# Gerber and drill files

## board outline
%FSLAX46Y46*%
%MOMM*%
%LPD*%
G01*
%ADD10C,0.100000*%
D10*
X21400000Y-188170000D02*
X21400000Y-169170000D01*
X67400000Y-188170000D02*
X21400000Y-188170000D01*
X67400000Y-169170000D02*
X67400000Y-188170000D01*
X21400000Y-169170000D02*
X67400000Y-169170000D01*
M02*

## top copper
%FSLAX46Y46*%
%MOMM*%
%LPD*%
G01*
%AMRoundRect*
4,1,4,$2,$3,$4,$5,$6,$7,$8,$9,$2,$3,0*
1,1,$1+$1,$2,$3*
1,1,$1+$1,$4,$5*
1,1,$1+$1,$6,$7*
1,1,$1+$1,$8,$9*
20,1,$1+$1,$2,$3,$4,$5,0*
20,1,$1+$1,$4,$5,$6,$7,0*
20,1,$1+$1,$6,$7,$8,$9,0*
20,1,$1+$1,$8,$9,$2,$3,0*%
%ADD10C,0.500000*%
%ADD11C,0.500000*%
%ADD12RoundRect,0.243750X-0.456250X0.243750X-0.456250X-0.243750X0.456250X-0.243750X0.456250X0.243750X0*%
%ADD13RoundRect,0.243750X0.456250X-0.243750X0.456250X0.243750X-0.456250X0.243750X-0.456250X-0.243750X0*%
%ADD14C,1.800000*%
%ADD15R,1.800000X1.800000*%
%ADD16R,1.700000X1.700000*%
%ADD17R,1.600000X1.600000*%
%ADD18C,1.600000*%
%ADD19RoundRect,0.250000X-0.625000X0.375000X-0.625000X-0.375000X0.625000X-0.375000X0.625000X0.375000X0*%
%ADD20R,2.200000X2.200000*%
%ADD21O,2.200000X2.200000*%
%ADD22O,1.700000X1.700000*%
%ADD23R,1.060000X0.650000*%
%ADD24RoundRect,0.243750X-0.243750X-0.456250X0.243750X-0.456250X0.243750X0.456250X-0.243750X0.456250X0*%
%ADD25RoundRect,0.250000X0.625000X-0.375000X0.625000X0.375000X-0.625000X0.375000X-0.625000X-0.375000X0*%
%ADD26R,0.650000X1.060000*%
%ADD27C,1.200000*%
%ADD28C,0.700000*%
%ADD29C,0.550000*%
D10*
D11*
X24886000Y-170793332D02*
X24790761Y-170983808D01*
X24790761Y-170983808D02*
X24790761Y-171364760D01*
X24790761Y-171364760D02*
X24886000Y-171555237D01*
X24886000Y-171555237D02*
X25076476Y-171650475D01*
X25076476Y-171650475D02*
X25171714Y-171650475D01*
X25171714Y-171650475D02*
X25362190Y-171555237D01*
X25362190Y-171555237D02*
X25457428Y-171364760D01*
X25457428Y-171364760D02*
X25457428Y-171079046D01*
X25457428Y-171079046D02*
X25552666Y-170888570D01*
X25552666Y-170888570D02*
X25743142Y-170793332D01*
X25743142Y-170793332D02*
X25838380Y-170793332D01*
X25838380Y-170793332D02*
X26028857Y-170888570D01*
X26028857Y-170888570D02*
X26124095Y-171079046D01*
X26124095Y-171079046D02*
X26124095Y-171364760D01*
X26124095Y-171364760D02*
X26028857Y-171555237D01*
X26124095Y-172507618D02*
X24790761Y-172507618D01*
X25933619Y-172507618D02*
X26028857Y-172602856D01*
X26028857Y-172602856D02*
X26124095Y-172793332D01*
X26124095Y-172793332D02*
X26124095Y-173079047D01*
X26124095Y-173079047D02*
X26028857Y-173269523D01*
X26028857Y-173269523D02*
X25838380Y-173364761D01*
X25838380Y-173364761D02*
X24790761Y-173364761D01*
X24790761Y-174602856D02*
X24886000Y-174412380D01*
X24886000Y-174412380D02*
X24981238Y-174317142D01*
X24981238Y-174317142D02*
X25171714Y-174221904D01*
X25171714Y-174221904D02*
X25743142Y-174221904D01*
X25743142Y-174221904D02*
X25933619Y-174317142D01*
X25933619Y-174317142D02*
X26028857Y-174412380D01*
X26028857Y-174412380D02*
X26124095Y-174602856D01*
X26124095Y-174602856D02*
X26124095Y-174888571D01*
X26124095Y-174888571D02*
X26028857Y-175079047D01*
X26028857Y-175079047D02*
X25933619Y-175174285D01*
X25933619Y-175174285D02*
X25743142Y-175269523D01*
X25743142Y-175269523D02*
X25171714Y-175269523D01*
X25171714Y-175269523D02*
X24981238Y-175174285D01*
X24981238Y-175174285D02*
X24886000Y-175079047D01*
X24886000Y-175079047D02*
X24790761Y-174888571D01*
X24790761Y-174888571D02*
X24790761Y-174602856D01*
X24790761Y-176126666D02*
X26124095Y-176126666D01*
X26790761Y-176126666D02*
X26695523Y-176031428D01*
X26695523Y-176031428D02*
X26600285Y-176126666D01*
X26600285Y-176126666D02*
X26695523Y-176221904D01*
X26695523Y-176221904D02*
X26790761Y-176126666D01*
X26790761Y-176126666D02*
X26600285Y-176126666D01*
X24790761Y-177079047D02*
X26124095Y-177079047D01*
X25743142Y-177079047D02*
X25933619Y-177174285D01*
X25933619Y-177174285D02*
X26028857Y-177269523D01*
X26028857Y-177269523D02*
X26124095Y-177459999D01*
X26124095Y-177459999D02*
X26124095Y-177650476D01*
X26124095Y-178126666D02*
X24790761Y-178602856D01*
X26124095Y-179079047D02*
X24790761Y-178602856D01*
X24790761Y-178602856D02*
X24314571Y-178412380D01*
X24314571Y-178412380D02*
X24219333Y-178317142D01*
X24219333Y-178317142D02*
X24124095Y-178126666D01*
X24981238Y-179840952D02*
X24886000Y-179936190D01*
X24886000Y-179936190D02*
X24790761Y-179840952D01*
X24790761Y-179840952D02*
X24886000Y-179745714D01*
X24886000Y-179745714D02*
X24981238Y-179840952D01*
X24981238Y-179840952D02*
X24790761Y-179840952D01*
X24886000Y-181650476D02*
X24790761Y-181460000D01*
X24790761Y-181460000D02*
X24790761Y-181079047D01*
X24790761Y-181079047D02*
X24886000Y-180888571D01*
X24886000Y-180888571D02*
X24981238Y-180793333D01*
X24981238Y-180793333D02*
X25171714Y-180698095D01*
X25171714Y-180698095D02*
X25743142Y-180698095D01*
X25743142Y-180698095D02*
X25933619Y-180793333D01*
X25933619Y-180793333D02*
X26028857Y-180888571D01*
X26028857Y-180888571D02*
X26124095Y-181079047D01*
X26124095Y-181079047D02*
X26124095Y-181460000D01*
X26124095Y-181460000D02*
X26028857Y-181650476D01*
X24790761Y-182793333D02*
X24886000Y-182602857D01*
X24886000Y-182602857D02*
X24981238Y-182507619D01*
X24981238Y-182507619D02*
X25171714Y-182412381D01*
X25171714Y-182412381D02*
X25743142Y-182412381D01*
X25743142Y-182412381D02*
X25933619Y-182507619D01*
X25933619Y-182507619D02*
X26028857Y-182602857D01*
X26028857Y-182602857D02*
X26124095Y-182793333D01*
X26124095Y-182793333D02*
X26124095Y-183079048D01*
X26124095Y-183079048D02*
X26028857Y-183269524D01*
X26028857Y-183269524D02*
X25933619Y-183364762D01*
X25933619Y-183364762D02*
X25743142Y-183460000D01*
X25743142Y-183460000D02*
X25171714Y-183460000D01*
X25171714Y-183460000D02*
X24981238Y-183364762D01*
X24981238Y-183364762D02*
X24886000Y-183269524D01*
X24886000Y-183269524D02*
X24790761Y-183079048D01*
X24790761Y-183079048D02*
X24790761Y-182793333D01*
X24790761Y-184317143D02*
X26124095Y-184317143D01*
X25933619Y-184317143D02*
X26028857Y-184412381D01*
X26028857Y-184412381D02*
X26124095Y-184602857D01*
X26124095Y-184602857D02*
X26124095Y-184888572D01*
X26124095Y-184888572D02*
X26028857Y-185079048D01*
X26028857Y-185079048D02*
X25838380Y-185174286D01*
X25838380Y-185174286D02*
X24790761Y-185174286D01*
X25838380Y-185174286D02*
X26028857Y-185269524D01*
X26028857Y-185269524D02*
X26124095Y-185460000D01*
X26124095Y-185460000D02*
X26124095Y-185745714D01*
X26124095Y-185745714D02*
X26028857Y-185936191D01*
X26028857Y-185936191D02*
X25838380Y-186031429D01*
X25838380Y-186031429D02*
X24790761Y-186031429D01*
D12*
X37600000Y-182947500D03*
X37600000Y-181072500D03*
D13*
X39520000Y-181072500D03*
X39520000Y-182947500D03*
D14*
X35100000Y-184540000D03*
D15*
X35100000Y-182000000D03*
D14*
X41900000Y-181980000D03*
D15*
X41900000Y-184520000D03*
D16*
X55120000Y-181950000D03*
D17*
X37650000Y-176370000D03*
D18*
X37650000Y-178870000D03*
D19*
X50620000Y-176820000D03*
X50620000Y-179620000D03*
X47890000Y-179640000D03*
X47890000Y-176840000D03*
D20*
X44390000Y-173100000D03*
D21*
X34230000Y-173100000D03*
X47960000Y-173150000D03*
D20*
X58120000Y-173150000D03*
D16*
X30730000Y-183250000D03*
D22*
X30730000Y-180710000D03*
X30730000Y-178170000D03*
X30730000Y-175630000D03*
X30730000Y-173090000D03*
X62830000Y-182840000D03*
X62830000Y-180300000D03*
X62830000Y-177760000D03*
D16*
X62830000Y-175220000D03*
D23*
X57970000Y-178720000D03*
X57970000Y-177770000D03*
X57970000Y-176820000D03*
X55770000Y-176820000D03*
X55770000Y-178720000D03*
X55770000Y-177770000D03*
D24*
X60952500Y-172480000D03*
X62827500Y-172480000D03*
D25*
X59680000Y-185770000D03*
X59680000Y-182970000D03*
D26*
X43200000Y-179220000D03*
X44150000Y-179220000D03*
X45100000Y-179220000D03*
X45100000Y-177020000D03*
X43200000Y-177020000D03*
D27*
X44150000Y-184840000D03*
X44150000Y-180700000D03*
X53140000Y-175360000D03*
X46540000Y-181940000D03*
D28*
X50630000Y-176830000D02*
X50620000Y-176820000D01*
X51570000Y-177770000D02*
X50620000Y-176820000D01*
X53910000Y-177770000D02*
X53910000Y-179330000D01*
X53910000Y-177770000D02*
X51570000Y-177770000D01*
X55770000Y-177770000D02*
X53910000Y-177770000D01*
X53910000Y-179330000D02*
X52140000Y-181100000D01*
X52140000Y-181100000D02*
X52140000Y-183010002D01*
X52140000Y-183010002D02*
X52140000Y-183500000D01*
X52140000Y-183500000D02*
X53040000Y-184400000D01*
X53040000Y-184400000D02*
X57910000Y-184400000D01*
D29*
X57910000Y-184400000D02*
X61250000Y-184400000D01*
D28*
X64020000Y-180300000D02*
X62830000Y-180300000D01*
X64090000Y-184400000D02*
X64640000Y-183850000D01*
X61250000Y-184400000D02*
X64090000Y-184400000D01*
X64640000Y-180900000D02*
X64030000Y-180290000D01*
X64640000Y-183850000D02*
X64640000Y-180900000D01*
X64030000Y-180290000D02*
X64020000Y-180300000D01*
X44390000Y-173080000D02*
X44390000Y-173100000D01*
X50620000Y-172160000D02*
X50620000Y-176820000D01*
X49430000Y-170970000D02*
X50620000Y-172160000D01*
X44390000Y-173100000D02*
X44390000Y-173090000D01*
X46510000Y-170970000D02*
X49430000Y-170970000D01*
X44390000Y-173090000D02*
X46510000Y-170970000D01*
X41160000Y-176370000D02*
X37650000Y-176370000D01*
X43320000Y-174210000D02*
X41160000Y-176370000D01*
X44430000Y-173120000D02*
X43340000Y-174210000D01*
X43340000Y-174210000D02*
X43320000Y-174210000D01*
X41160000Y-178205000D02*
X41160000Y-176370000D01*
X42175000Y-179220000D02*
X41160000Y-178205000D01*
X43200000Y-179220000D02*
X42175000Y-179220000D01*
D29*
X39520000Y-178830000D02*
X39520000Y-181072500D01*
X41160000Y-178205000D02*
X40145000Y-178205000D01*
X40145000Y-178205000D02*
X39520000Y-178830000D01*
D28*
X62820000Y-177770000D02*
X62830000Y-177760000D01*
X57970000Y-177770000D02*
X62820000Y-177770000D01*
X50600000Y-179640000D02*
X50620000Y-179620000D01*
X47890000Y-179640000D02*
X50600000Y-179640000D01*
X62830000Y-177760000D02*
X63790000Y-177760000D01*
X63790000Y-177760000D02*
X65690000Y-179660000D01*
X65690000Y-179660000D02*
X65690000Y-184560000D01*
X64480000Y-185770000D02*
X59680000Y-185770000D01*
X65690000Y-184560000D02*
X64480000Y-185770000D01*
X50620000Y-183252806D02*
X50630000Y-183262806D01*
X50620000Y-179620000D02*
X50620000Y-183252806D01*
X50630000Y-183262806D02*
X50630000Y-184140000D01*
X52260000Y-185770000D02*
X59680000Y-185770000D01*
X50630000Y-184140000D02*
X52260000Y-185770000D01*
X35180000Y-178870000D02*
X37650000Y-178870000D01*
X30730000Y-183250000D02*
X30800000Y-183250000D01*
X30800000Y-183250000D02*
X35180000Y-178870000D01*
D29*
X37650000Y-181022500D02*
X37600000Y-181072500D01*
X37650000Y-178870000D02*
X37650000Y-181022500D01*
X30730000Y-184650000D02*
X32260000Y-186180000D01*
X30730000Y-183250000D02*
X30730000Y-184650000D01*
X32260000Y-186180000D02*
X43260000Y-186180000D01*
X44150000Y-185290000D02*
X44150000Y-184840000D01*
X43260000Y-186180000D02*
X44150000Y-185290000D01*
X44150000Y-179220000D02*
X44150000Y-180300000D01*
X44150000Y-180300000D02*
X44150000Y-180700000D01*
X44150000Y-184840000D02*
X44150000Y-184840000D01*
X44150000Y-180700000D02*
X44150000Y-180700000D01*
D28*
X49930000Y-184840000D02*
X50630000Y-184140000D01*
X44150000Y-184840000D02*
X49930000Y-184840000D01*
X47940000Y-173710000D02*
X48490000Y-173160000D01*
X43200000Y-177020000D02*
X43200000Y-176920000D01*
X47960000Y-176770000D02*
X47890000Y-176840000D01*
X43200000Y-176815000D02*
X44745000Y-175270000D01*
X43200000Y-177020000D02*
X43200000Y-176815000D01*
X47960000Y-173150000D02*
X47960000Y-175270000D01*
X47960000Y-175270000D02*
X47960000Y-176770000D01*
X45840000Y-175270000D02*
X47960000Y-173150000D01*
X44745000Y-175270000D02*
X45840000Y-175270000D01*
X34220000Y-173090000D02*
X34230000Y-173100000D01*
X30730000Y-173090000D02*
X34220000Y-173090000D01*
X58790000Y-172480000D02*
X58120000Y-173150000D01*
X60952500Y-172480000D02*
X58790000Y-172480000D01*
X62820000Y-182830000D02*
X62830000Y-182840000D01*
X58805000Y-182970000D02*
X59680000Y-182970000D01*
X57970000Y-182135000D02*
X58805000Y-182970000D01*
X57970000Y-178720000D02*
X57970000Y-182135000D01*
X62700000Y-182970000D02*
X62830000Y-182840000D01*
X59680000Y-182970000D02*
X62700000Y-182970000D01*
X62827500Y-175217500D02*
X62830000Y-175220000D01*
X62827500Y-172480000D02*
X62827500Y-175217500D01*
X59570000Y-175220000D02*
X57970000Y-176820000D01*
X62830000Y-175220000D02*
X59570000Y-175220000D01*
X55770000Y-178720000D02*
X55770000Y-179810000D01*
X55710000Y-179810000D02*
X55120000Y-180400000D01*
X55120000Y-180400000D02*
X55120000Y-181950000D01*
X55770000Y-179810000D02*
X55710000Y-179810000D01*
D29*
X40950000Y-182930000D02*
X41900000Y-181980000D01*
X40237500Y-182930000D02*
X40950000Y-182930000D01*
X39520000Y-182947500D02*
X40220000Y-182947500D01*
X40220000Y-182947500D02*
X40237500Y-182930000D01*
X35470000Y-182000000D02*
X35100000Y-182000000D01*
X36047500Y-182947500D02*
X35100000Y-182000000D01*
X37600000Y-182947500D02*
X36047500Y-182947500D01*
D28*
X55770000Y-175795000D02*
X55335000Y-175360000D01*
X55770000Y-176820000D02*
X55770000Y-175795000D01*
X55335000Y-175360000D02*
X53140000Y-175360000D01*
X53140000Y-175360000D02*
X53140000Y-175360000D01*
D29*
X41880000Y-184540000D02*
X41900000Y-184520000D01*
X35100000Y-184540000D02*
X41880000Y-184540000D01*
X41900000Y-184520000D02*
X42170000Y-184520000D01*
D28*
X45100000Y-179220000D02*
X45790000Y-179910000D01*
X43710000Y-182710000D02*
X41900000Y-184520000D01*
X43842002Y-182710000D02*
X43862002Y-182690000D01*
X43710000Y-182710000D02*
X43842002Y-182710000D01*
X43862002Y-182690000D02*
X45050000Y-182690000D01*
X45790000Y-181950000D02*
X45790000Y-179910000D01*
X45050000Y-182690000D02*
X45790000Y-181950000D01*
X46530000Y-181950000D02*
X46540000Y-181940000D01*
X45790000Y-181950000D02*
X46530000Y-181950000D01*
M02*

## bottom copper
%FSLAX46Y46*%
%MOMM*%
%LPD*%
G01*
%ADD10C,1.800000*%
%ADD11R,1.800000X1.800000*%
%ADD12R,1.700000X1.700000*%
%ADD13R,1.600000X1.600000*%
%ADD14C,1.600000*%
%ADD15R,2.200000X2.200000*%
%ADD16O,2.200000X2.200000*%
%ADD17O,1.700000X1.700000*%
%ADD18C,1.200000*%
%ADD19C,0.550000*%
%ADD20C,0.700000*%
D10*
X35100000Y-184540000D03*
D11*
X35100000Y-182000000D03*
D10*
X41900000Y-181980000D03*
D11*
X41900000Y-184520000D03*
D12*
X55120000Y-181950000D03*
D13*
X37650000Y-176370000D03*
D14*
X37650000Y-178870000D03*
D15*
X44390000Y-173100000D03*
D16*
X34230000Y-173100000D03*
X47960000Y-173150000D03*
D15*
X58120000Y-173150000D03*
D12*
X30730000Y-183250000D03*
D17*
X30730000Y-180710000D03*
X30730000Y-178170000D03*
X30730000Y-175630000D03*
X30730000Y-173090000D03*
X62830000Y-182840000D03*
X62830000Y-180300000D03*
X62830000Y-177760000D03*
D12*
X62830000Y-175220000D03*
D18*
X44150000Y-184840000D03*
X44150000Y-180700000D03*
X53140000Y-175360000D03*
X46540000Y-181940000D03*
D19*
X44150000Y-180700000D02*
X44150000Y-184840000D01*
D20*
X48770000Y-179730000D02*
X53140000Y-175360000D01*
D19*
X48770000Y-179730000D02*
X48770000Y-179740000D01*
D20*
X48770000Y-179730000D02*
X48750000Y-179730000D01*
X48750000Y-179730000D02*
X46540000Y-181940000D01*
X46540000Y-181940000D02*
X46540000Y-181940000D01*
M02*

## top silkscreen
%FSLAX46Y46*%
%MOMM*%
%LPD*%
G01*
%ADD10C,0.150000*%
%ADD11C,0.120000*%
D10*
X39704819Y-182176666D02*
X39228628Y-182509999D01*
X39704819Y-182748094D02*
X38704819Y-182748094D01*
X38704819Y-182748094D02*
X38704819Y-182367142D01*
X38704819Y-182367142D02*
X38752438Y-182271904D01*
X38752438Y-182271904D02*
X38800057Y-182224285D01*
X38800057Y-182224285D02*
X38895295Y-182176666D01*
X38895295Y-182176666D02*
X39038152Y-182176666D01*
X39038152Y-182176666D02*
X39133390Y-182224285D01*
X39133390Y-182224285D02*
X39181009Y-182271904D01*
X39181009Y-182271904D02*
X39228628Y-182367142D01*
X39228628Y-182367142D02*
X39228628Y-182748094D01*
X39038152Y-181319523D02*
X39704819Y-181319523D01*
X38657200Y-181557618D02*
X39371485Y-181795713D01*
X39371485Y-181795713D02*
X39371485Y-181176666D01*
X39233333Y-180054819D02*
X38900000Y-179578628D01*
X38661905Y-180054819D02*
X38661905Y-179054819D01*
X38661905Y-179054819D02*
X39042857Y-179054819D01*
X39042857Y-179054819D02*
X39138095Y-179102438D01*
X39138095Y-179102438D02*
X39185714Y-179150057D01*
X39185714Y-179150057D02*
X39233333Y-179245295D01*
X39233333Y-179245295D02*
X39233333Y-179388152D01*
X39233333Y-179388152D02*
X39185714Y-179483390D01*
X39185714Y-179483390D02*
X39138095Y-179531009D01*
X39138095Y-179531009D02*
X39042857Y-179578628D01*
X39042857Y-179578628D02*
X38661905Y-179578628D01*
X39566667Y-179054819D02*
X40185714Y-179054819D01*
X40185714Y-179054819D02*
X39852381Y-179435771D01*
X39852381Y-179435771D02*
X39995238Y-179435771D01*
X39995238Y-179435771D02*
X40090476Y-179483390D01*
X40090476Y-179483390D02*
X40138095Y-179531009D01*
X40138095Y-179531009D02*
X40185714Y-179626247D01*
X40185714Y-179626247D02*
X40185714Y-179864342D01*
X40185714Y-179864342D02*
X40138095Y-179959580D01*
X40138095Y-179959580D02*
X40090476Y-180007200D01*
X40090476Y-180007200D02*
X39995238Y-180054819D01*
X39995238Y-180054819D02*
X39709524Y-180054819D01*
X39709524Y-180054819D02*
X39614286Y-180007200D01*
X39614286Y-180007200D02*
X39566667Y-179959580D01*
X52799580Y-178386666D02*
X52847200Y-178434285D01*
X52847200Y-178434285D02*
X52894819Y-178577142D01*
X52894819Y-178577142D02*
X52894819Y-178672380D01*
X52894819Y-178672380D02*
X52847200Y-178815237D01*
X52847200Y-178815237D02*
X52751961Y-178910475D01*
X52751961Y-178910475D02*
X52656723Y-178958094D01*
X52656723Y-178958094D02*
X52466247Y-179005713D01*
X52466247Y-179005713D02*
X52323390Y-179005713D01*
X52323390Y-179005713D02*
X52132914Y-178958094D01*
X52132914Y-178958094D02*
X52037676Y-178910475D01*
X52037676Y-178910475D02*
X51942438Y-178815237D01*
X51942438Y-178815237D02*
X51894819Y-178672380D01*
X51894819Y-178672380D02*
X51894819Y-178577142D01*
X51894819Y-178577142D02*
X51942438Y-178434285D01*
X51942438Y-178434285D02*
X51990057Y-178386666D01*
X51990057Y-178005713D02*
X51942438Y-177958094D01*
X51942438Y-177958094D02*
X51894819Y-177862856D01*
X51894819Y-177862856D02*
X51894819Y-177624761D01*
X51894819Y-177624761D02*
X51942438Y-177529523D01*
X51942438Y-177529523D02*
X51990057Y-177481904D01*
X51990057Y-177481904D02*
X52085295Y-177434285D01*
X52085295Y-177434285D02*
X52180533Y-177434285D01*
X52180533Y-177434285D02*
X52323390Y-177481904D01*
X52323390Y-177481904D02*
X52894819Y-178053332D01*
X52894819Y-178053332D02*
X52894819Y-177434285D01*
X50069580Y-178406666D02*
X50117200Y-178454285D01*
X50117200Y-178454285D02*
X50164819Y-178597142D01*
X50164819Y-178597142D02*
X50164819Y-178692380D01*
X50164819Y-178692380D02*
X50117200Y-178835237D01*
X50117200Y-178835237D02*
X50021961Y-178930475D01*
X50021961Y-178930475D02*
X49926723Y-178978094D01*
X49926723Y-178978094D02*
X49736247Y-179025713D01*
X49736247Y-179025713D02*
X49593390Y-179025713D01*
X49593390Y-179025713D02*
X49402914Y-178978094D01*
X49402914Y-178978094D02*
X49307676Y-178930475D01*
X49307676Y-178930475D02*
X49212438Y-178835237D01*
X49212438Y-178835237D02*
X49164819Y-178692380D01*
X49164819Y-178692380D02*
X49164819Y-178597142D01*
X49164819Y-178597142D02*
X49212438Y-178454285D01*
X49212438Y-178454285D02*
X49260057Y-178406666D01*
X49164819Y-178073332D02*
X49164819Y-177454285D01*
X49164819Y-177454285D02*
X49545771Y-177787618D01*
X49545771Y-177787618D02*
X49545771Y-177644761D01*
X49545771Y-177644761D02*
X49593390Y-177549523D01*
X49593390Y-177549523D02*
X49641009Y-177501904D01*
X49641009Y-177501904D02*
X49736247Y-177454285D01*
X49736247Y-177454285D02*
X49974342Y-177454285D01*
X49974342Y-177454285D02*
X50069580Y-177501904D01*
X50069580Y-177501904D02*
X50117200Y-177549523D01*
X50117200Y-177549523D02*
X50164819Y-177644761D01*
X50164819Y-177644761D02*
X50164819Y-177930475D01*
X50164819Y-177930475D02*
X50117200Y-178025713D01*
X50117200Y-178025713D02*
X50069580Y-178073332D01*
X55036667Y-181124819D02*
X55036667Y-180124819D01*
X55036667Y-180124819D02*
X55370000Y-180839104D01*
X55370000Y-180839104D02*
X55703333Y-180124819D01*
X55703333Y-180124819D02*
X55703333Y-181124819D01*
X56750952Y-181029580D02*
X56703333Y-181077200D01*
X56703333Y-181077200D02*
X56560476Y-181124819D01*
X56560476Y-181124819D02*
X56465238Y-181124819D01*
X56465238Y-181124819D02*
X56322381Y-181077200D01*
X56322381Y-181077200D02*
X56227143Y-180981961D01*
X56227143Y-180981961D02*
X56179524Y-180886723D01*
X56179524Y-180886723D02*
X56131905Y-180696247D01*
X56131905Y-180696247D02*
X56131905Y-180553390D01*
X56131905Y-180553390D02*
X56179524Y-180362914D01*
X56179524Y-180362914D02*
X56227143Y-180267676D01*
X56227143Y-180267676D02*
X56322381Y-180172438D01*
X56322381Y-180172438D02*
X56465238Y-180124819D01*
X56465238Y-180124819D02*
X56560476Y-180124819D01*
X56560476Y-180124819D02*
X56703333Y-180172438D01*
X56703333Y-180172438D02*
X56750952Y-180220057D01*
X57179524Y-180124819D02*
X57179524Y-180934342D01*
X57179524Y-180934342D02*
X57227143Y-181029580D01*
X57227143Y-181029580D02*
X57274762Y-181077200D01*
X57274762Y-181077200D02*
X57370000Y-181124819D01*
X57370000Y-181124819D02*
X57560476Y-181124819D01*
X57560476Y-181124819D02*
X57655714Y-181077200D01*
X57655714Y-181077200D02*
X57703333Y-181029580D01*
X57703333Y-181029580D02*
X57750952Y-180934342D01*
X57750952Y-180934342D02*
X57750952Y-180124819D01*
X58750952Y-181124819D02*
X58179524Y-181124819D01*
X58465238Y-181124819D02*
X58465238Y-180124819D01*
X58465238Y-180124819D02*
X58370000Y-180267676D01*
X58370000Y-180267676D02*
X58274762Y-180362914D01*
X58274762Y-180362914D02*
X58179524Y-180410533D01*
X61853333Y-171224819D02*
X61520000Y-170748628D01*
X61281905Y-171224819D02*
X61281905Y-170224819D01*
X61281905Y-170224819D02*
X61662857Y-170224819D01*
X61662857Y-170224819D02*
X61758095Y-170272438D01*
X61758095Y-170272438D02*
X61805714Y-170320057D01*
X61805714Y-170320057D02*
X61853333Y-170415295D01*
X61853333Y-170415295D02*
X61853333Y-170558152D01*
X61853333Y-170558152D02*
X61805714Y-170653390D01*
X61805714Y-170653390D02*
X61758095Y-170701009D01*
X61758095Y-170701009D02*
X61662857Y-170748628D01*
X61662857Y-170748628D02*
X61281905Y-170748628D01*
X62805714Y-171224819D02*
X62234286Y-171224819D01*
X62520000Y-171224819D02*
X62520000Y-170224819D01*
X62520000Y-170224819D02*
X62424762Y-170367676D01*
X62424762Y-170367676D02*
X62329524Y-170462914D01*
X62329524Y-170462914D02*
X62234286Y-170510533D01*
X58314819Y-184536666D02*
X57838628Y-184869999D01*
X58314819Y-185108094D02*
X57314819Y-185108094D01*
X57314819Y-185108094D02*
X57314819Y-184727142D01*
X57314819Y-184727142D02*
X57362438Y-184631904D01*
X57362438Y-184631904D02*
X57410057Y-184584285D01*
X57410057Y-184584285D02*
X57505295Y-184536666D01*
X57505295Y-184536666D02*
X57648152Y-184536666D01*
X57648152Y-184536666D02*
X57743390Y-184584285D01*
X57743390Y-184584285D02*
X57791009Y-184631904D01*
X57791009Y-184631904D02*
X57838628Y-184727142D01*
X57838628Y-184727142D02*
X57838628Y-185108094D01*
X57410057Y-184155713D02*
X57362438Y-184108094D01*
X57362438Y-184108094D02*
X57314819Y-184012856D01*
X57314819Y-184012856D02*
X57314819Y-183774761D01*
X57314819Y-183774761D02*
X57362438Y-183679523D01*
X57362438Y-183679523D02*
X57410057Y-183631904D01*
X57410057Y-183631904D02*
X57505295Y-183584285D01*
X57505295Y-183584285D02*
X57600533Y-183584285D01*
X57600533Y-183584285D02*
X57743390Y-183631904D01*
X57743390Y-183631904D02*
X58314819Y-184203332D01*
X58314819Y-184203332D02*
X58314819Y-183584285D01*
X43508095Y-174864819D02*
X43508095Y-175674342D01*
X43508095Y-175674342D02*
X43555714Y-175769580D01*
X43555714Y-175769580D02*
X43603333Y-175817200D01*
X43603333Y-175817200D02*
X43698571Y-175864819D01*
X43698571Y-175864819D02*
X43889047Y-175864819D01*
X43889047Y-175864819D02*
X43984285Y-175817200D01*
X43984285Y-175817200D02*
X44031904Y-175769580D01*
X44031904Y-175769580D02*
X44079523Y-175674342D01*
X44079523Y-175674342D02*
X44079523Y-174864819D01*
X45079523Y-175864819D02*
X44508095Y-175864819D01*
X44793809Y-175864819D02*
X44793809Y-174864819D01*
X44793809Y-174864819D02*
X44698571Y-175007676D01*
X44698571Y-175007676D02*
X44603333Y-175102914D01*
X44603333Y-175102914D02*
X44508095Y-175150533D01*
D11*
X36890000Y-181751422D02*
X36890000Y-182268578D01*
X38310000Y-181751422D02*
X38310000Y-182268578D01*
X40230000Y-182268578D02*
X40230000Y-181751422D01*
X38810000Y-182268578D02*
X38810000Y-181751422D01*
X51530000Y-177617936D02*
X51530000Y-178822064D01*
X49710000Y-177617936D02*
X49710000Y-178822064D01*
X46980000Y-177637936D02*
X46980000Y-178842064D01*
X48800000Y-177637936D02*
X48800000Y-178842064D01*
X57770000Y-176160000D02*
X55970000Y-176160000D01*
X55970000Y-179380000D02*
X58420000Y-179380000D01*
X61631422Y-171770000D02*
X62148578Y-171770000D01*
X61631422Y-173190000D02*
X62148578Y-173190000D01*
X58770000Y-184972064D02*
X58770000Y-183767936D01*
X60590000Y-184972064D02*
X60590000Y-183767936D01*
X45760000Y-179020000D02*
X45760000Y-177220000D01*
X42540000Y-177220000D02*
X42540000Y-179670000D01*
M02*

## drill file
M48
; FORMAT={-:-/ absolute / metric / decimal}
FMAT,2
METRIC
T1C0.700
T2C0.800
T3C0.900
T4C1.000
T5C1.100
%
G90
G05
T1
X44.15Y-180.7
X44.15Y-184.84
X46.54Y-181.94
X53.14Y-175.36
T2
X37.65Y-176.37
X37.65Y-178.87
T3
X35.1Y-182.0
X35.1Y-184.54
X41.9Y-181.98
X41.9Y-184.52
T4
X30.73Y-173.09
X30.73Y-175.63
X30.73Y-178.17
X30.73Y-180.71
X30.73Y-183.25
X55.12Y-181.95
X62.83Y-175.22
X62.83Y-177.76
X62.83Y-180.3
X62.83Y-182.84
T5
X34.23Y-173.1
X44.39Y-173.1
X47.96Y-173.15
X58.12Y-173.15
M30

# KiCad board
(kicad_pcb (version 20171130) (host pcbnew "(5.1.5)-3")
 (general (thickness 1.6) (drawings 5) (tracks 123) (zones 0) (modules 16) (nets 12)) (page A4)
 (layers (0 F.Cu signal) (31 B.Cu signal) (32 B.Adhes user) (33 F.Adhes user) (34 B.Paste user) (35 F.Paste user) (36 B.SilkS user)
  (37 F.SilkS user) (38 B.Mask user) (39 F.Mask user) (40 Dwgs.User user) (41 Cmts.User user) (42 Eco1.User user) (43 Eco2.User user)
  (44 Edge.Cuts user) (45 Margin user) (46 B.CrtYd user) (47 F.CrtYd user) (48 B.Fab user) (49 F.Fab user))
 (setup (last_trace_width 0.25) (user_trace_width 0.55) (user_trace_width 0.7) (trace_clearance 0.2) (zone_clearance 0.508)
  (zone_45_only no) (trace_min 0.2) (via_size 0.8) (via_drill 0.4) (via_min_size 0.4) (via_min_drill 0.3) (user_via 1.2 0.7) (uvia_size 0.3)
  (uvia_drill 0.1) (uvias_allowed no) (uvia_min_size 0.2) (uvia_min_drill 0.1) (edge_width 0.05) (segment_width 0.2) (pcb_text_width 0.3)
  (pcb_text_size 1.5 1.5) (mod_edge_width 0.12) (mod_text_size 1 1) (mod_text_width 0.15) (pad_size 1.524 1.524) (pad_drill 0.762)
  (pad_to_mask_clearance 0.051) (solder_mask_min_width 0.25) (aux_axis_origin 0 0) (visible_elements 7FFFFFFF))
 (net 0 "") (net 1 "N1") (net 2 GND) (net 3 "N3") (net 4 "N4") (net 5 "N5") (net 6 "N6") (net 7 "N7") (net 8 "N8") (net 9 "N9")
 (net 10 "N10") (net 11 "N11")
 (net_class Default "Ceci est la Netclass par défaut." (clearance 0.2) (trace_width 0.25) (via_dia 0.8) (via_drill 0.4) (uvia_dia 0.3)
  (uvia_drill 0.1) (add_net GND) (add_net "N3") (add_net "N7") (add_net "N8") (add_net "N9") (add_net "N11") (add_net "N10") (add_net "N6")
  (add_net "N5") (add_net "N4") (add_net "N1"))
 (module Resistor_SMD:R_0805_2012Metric (layer F.Cu) (at 37.6 182.01 270)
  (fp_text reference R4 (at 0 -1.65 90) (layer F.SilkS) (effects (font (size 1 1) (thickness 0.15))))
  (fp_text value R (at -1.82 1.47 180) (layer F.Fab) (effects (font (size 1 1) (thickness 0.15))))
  (fp_line (start -0.258578 0.71) (end 0.258578 0.71) (layer F.SilkS) (width 0.12))
  (fp_line (start -0.258578 -0.71) (end 0.258578 -0.71) (layer F.SilkS) (width 0.12))
  (pad 2 smd roundrect (at 0.9375 0 270) (size 0.975 1.4) (layers F.Cu F.Paste F.Mask) (roundrect_rratio 0.25) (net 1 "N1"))
  (pad 1 smd roundrect (at -0.9375 0 270) (size 0.975 1.4) (layers F.Cu F.Paste F.Mask) (roundrect_rratio 0.25) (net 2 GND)))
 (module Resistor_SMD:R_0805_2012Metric (layer F.Cu) (at 39.52 182.01 90)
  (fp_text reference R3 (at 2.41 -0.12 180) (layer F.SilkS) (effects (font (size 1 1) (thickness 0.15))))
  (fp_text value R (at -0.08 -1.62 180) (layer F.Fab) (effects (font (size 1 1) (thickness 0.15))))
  (fp_line (start -0.258578 0.71) (end 0.258578 0.71) (layer F.SilkS) (width 0.12))
  (fp_line (start -0.258578 -0.71) (end 0.258578 -0.71) (layer F.SilkS) (width 0.12))
  (pad 2 smd roundrect (at 0.9375 0 90) (size 0.975 1.4) (layers F.Cu F.Paste F.Mask) (roundrect_rratio 0.25) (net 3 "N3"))
  (pad 1 smd roundrect (at -0.9375 0 90) (size 0.975 1.4) (layers F.Cu F.Paste F.Mask) (roundrect_rratio 0.25) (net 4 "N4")))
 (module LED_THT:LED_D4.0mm (layer B.Cu) (at 35.1 182 270)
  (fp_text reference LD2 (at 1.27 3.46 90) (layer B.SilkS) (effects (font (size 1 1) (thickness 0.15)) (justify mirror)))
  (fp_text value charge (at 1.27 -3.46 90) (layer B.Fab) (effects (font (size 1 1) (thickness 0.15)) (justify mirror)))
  (pad 2 thru_hole circle (at 2.54 0 270) (size 1.8 1.8) (drill 0.9) (layers *.Cu *.Mask) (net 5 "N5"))
  (pad 1 thru_hole rect (at 0 0 270) (size 1.8 1.8) (drill 0.9) (layers *.Cu *.Mask) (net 1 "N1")))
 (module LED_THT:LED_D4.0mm (layer B.Cu) (at 41.9 184.52 90)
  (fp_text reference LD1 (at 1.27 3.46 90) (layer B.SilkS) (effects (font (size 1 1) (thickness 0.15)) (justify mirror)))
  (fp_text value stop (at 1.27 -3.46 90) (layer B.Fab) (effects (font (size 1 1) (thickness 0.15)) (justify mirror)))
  (pad 2 thru_hole circle (at 2.54 0 90) (size 1.8 1.8) (drill 0.9) (layers *.Cu *.Mask) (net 4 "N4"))
  (pad 1 thru_hole rect (at 0 0 90) (size 1.8 1.8) (drill 0.9) (layers *.Cu *.Mask) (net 5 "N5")))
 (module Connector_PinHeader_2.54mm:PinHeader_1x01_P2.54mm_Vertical (layer B.Cu) (at 55.12 181.95)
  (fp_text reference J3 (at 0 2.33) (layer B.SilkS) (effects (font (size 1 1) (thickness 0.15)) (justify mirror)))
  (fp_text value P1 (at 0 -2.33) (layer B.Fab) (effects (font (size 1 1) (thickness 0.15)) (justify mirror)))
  (pad 1 thru_hole rect (at 0 0) (size 1.7 1.7) (drill 1) (layers *.Cu *.Mask) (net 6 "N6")))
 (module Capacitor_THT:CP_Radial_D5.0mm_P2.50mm (layer B.Cu) (at 37.65 176.37 270)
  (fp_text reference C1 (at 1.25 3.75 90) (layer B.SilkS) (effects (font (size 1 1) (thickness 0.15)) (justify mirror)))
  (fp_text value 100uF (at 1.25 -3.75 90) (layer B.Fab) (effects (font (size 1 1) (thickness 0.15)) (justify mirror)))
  (pad 1 thru_hole rect (at 0 0 270) (size 1.6 1.6) (drill 0.8) (layers *.Cu *.Mask) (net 3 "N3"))
  (pad 2 thru_hole circle (at 2.5 0 270) (size 1.6 1.6) (drill 0.8) (layers *.Cu *.Mask) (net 2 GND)))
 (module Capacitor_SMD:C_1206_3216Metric (layer F.Cu) (at 50.62 178.22 270)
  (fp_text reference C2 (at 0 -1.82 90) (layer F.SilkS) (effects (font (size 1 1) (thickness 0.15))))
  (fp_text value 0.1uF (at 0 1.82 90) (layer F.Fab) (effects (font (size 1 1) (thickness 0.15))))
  (fp_line (start -0.602064 -0.91) (end 0.602064 -0.91) (layer F.SilkS) (width 0.12))
  (fp_line (start -0.602064 0.91) (end 0.602064 0.91) (layer F.SilkS) (width 0.12))
  (pad 1 smd roundrect (at -1.4 0 270) (size 1.25 1.75) (layers F.Cu F.Paste F.Mask) (roundrect_rratio 0.2) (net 3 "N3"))
  (pad 2 smd roundrect (at 1.4 0 270) (size 1.25 1.75) (layers F.Cu F.Paste F.Mask) (roundrect_rratio 0.2) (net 2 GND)))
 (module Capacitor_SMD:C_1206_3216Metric (layer F.Cu) (at 47.89 178.24 270)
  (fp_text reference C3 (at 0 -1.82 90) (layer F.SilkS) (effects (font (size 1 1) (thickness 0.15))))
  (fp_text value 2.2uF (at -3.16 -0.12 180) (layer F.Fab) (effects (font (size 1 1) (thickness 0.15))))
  (fp_line (start -0.602064 0.91) (end 0.602064 0.91) (layer F.SilkS) (width 0.12))
  (fp_line (start -0.602064 -0.91) (end 0.602064 -0.91) (layer F.SilkS) (width 0.12))
  (pad 2 smd roundrect (at 1.4 0 270) (size 1.25 1.75) (layers F.Cu F.Paste F.Mask) (roundrect_rratio 0.2) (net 2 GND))
  (pad 1 smd roundrect (at -1.4 0 270) (size 1.25 1.75) (layers F.Cu F.Paste F.Mask) (roundrect_rratio 0.2) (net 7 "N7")))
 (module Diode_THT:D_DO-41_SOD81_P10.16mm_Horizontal (layer B.Cu) (at 44.39 173.1 180)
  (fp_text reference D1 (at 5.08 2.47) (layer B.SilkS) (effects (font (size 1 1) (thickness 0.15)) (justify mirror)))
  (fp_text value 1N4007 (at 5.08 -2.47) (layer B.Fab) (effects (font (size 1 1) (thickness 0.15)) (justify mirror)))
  (pad 1 thru_hole rect (at 0 0 180) (size 2.2 2.2) (drill 1.1) (layers *.Cu *.Mask) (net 3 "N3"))
  (pad 2 thru_hole oval (at 10.16 0 180) (size 2.2 2.2) (drill 1.1) (layers *.Cu *.Mask) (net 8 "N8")))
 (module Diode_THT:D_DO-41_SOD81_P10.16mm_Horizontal (layer B.Cu) (at 58.12 173.15 180)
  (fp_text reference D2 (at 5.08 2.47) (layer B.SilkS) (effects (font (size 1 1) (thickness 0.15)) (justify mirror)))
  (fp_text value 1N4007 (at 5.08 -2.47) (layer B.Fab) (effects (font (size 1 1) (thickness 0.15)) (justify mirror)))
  (pad 2 thru_hole oval (at 10.16 0 180) (size 2.2 2.2) (drill 1.1) (layers *.Cu *.Mask) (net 7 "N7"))
  (pad 1 thru_hole rect (at 0 0 180) (size 2.2 2.2) (drill 1.1) (layers *.Cu *.Mask) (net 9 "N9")))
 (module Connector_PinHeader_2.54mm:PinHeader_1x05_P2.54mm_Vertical (layer B.Cu) (at 30.73 183.25)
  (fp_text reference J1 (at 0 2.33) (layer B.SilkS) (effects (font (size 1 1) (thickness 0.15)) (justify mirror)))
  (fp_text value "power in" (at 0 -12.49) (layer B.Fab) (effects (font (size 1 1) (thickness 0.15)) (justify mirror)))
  (pad 1 thru_hole rect (at 0 0) (size 1.7 1.7) (drill 1) (layers *.Cu *.Mask) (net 2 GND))
  (pad 2 thru_hole oval (at 0 -2.54) (size 1.7 1.7) (drill 1) (layers *.Cu *.Mask))
  (pad 3 thru_hole oval (at 0 -5.08) (size 1.7 1.7) (drill 1) (layers *.Cu *.Mask))
  (pad 4 thru_hole oval (at 0 -7.62) (size 1.7 1.7) (drill 1) (layers *.Cu *.Mask))
  (pad 5 thru_hole oval (at 0 -10.16) (size 1.7 1.7) (drill 1) (layers *.Cu *.Mask) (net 8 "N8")))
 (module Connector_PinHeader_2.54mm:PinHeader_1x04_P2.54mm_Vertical (layer B.Cu) (at 62.83 175.22 180)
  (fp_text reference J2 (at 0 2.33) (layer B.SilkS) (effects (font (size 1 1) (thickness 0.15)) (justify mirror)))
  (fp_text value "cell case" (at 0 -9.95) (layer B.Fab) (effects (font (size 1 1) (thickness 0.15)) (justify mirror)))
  (pad 4 thru_hole oval (at 0 -7.62 180) (size 1.7 1.7) (drill 1) (layers *.Cu *.Mask) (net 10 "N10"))
  (pad 3 thru_hole oval (at 0 -5.08 180) (size 1.7 1.7) (drill 1) (layers *.Cu *.Mask) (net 3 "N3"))
  (pad 2 thru_hole oval (at 0 -2.54 180) (size 1.7 1.7) (drill 1) (layers *.Cu *.Mask) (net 2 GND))
  (pad 1 thru_hole rect (at 0 0 180) (size 1.7 1.7) (drill 1) (layers *.Cu *.Mask) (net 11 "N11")))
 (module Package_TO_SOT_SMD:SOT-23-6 (layer F.Cu) (at 56.87 177.77 180)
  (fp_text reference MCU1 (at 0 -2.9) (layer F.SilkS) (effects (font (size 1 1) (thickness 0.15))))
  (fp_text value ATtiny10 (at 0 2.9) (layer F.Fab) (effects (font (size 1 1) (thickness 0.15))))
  (fp_line (start -0.9 1.61) (end 0.9 1.61) (layer F.SilkS) (width 0.12))
  (fp_line (start 0.9 -1.61) (end -1.55 -1.61) (layer F.SilkS) (width 0.12))
  (pad 1 smd rect (at -1.1 -0.95 180) (size 1.06 0.65) (layers F.Cu F.Paste F.Mask) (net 10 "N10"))
  (pad 2 smd rect (at -1.1 0 180) (size 1.06 0.65) (layers F.Cu F.Paste F.Mask) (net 2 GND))
  (pad 3 smd rect (at -1.1 0.95 180) (size 1.06 0.65) (layers F.Cu F.Paste F.Mask) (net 11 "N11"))
  (pad 4 smd rect (at 1.1 0.95 180) (size 1.06 0.65) (layers F.Cu F.Paste F.Mask) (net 5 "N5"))
  (pad 6 smd rect (at 1.1 -0.95 180) (size 1.06 0.65) (layers F.Cu F.Paste F.Mask) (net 6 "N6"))
  (pad 5 smd rect (at 1.1 0 180) (size 1.06 0.65) (layers F.Cu F.Paste F.Mask) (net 3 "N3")))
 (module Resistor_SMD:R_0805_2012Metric (layer F.Cu) (at 61.89 172.48)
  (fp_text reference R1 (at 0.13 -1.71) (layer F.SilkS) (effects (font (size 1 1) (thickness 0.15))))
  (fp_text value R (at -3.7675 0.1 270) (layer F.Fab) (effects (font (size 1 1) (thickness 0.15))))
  (fp_line (start -0.258578 -0.71) (end 0.258578 -0.71) (layer F.SilkS) (width 0.12))
  (fp_line (start -0.258578 0.71) (end 0.258578 0.71) (layer F.SilkS) (width 0.12))
  (pad 1 smd roundrect (at -0.9375 0) (size 0.975 1.4) (layers F.Cu F.Paste F.Mask) (roundrect_rratio 0.25) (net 9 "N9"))
  (pad 2 smd roundrect (at 0.9375 0) (size 0.975 1.4) (layers F.Cu F.Paste F.Mask) (roundrect_rratio 0.25) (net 11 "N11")))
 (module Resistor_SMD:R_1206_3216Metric (layer F.Cu) (at 59.68 184.37 90)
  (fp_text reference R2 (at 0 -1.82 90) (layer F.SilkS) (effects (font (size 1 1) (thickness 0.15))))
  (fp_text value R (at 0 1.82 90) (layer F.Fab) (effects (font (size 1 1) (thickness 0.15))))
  (fp_line (start -0.602064 -0.91) (end 0.602064 -0.91) (layer F.SilkS) (width 0.12))
  (fp_line (start -0.602064 0.91) (end 0.602064 0.91) (layer F.SilkS) (width 0.12))
  (pad 1 smd roundrect (at -1.4 0 90) (size 1.25 1.75) (layers F.Cu F.Paste F.Mask) (roundrect_rratio 0.2) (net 2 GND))
  (pad 2 smd roundrect (at 1.4 0 90) (size 1.25 1.75) (layers F.Cu F.Paste F.Mask) (roundrect_rratio 0.2) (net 10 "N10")))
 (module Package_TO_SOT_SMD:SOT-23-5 (layer F.Cu) (at 44.15 178.12 90)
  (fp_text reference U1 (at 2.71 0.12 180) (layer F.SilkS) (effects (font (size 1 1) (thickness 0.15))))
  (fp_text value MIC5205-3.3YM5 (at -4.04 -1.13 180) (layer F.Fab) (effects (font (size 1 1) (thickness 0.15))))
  (fp_line (start -0.9 1.61) (end 0.9 1.61) (layer F.SilkS) (width 0.12))
  (fp_line (start 0.9 -1.61) (end -1.55 -1.61) (layer F.SilkS) (width 0.12))
  (pad 1 smd rect (at -1.1 -0.95 90) (size 1.06 0.65) (layers F.Cu F.Paste F.Mask) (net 3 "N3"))
  (pad 2 smd rect (at -1.1 0 90) (size 1.06 0.65) (layers F.Cu F.Paste F.Mask) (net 2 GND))
  (pad 3 smd rect (at -1.1 0.95 90) (size 1.06 0.65) (layers F.Cu F.Paste F.Mask) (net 5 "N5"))
  (pad 4 smd rect (at 1.1 0.95 90) (size 1.06 0.65) (layers F.Cu F.Paste F.Mask))
  (pad 5 smd rect (at 1.1 -0.95 90) (size 1.06 0.65) (layers F.Cu F.Paste F.Mask) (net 7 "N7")))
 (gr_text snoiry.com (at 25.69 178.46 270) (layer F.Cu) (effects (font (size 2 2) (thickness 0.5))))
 (gr_line (start 21.4 188.17) (end 21.4 169.17) (layer Edge.Cuts) (width 0.1))
 (gr_line (start 67.4 188.17) (end 21.4 188.17) (layer Edge.Cuts) (width 0.1))
 (gr_line (start 67.4 169.17) (end 67.4 188.17) (layer Edge.Cuts) (width 0.1))
 (gr_line (start 21.4 169.17) (end 67.4 169.17) (layer Edge.Cuts) (width 0.1))
 (segment (start 50.63 176.83) (end 50.62 176.82) (width 0.7) (layer F.Cu) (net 3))
 (segment (start 51.57 177.77) (end 50.62 176.82) (width 0.7) (layer F.Cu) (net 3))
 (segment (start 53.91 177.77) (end 53.91 179.33) (width 0.7) (layer F.Cu) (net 3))
 (segment (start 53.91 177.77) (end 51.57 177.77) (width 0.7) (layer F.Cu) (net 3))
 (segment (start 55.77 177.77) (end 53.91 177.77) (width 0.7) (layer F.Cu) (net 3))
 (segment (start 53.91 179.33) (end 52.14 181.1) (width 0.7) (layer F.Cu) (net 3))
 (segment (start 52.14 181.1) (end 52.14 183.010002) (width 0.7) (layer F.Cu) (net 3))
 (segment (start 52.14 183.010002) (end 52.14 183.5) (width 0.7) (layer F.Cu) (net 3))
 (segment (start 52.14 183.5) (end 53.04 184.4) (width 0.7) (layer F.Cu) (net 3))
 (segment (start 53.04 184.4) (end 57.91 184.4) (width 0.7) (layer F.Cu) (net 3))
 (segment (start 57.91 184.4) (end 61.25 184.4) (width 0.55) (layer F.Cu) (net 3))
 (segment (start 64.02 180.3) (end 62.83 180.3) (width 0.7) (layer F.Cu) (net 3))
 (segment (start 64.09 184.4) (end 64.64 183.85) (width 0.7) (layer F.Cu) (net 3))
 (segment (start 61.25 184.4) (end 64.09 184.4) (width 0.7) (layer F.Cu) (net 3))
 (segment (start 64.64 180.9) (end 64.03 180.29) (width 0.7) (layer F.Cu) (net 3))
 (segment (start 64.64 183.85) (end 64.64 180.9) (width 0.7) (layer F.Cu) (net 3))
 (segment (start 64.03 180.29) (end 64.02 180.3) (width 0.7) (layer F.Cu) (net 3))
 (segment (start 44.39 173.08) (end 44.39 173.1) (width 0.7) (layer F.Cu) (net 3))
 (segment (start 50.62 172.16) (end 50.62 176.82) (width 0.7) (layer F.Cu) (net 3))
 (segment (start 49.43 170.97) (end 50.62 172.16) (width 0.7) (layer F.Cu) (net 3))
 (segment (start 44.39 173.1) (end 44.39 173.09) (width 0.7) (layer F.Cu) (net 3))
 (segment (start 46.51 170.97) (end 49.43 170.97) (width 0.7) (layer F.Cu) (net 3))
 (segment (start 44.39 173.09) (end 46.51 170.97) (width 0.7) (layer F.Cu) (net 3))
 (segment (start 41.16 176.37) (end 37.65 176.37) (width 0.7) (layer F.Cu) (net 3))
 (segment (start 43.32 174.21) (end 41.16 176.37) (width 0.7) (layer F.Cu) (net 3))
 (segment (start 44.43 173.12) (end 43.34 174.21) (width 0.7) (layer F.Cu) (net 3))
 (segment (start 43.34 174.21) (end 43.32 174.21) (width 0.7) (layer F.Cu) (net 3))
 (segment (start 41.16 178.205) (end 41.16 176.37) (width 0.7) (layer F.Cu) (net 3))
 (segment (start 42.175 179.22) (end 41.16 178.205) (width 0.7) (layer F.Cu) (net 3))
 (segment (start 43.2 179.22) (end 42.175 179.22) (width 0.7) (layer F.Cu) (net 3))
 (segment (start 39.52 178.83) (end 39.52 181.0725) (width 0.55) (layer F.Cu) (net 3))
 (segment (start 41.16 178.205) (end 40.145 178.205) (width 0.55) (layer F.Cu) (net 3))
 (segment (start 40.145 178.205) (end 39.52 178.83) (width 0.55) (layer F.Cu) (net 3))
 (segment (start 62.82 177.77) (end 62.83 177.76) (width 0.7) (layer F.Cu) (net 2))
 (segment (start 57.97 177.77) (end 62.82 177.77) (width 0.7) (layer F.Cu) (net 2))
 (segment (start 50.6 179.64) (end 50.62 179.62) (width 0.7) (layer F.Cu) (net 2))
 (segment (start 47.89 179.64) (end 50.6 179.64) (width 0.7) (layer F.Cu) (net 2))
 (segment (start 62.83 177.76) (end 63.79 177.76) (width 0.7) (layer F.Cu) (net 2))
 (segment (start 63.79 177.76) (end 65.69 179.66) (width 0.7) (layer F.Cu) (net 2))
 (segment (start 65.69 179.66) (end 65.69 184.56) (width 0.7) (layer F.Cu) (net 2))
 (segment (start 64.48 185.77) (end 59.68 185.77) (width 0.7) (layer F.Cu) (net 2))
 (segment (start 65.69 184.56) (end 64.48 185.77) (width 0.7) (layer F.Cu) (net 2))
 (segment (start 50.62 183.252806) (end 50.63 183.262806) (width 0.7) (layer F.Cu) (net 2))
 (segment (start 50.62 179.62) (end 50.62 183.252806) (width 0.7) (layer F.Cu) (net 2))
 (segment (start 50.63 183.262806) (end 50.63 184.14) (width 0.7) (layer F.Cu) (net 2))
 (segment (start 52.26 185.77) (end 59.68 185.77) (width 0.7) (layer F.Cu) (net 2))
 (segment (start 50.63 184.14) (end 52.26 185.77) (width 0.7) (layer F.Cu) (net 2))
 (segment (start 35.18 178.87) (end 37.65 178.87) (width 0.7) (layer F.Cu) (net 2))
 (segment (start 30.73 183.25) (end 30.8 183.25) (width 0.7) (layer F.Cu) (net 2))
 (segment (start 30.8 183.25) (end 35.18 178.87) (width 0.7) (layer F.Cu) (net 2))
 (segment (start 37.65 181.0225) (end 37.6 181.0725) (width 0.55) (layer F.Cu) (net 2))
 (segment (start 37.65 178.87) (end 37.65 181.0225) (width 0.55) (layer F.Cu) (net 2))
 (segment (start 30.73 184.65) (end 32.26 186.18) (width 0.55) (layer F.Cu) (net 2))
 (segment (start 30.73 183.25) (end 30.73 184.65) (width 0.55) (layer F.Cu) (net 2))
 (segment (start 32.26 186.18) (end 43.26 186.18) (width 0.55) (layer F.Cu) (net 2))
 (segment (start 44.15 185.29) (end 44.15 184.84) (width 0.55) (layer F.Cu) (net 2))
 (segment (start 43.26 186.18) (end 44.15 185.29) (width 0.55) (layer F.Cu) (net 2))
 (segment (start 44.15 179.22) (end 44.15 180.3) (width 0.55) (layer F.Cu) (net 2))
 (segment (start 44.15 180.3) (end 44.15 180.7) (width 0.55) (layer F.Cu) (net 2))
 (segment (start 44.15 184.84) (end 44.15 184.84) (width 0.55) (layer F.Cu) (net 2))
 (via (at 44.15 184.84) (size 1.2) (drill 0.7) (layers F.Cu B.Cu) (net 2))
 (segment (start 44.15 180.7) (end 44.15 180.7) (width 0.55) (layer F.Cu) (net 2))
 (via (at 44.15 180.7) (size 1.2) (drill 0.7) (layers F.Cu B.Cu) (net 2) (status 1000000))
 (segment (start 44.15 180.7) (end 44.15 184.84) (width 0.55) (layer B.Cu) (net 2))
 (segment (start 49.93 184.84) (end 50.63 184.14) (width 0.7) (layer F.Cu) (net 2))
 (segment (start 44.15 184.84) (end 49.93 184.84) (width 0.7) (layer F.Cu) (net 2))
 (segment (start 47.94 173.71) (end 48.49 173.16) (width 0.7) (layer F.Cu) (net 7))
 (segment (start 43.2 177.02) (end 43.2 176.92) (width 0.7) (layer F.Cu) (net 7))
 (segment (start 47.96 176.77) (end 47.89 176.84) (width 0.7) (layer F.Cu) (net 7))
 (segment (start 43.2 176.815) (end 44.745 175.27) (width 0.7) (layer F.Cu) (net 7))
 (segment (start 43.2 177.02) (end 43.2 176.815) (width 0.7) (layer F.Cu) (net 7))
 (segment (start 47.96 173.15) (end 47.96 175.27) (width 0.7) (layer F.Cu) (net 7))
 (segment (start 47.96 175.27) (end 47.96 176.77) (width 0.7) (layer F.Cu) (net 7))
 (segment (start 45.84 175.27) (end 47.96 173.15) (width 0.7) (layer F.Cu) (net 7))
 (segment (start 44.745 175.27) (end 45.84 175.27) (width 0.7) (layer F.Cu) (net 7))
 (segment (start 34.22 173.09) (end 34.23 173.1) (width 0.7) (layer F.Cu) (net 8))
 (segment (start 30.73 173.09) (end 34.22 173.09) (width 0.7) (layer F.Cu) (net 8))
 (segment (start 58.79 172.48) (end 58.12 173.15) (width 0.7) (layer F.Cu) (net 9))
 (segment (start 60.9525 172.48) (end 58.79 172.48) (width 0.7) (layer F.Cu) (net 9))
 (segment (start 62.82 182.83) (end 62.83 182.84) (width 0.7) (layer F.Cu) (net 10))
 (segment (start 58.805 182.97) (end 59.68 182.97) (width 0.7) (layer F.Cu) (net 10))
 (segment (start 57.97 182.135) (end 58.805 182.97) (width 0.7) (layer F.Cu) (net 10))
 (segment (start 57.97 178.72) (end 57.97 182.135) (width 0.7) (layer F.Cu) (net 10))
 (segment (start 62.7 182.97) (end 62.83 182.84) (width 0.7) (layer F.Cu) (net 10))
 (segment (start 59.68 182.97) (end 62.7 182.97) (width 0.7) (layer F.Cu) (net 10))
 (segment (start 62.8275 175.2175) (end 62.83 175.22) (width 0.7) (layer F.Cu) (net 11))
 (segment (start 62.8275 172.48) (end 62.8275 175.2175) (width 0.7) (layer F.Cu) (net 11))
 (segment (start 59.57 175.22) (end 57.97 176.82) (width 0.7) (layer F.Cu) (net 11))
 (segment (start 62.83 175.22) (end 59.57 175.22) (width 0.7) (layer F.Cu) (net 11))
 (segment (start 55.77 178.72) (end 55.77 179.81) (width 0.7) (layer F.Cu) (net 6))
 (segment (start 55.71 179.81) (end 55.12 180.4) (width 0.7) (layer F.Cu) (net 6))
 (segment (start 55.12 180.4) (end 55.12 181.95) (width 0.7) (layer F.Cu) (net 6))
 (segment (start 55.77 179.81) (end 55.71 179.81) (width 0.7) (layer F.Cu) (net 6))
 (segment (start 40.95 182.93) (end 41.9 181.98) (width 0.55) (layer F.Cu) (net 4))
 (segment (start 40.2375 182.93) (end 40.95 182.93) (width 0.55) (layer F.Cu) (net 4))
 (segment (start 39.52 182.9475) (end 40.22 182.9475) (width 0.55) (layer F.Cu) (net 4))
 (segment (start 40.22 182.9475) (end 40.2375 182.93) (width 0.55) (layer F.Cu) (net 4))
 (segment (start 35.47 182) (end 35.1 182) (width 0.55) (layer F.Cu) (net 1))
 (segment (start 36.0475 182.9475) (end 35.1 182) (width 0.55) (layer F.Cu) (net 1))
 (segment (start 37.6 182.9475) (end 36.0475 182.9475) (width 0.55) (layer F.Cu) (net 1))
 (segment (start 55.77 175.795) (end 55.335 175.36) (width 0.7) (layer F.Cu) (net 5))
 (segment (start 55.77 176.82) (end 55.77 175.795) (width 0.7) (layer F.Cu) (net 5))
 (segment (start 55.335 175.36) (end 53.14 175.36) (width 0.7) (layer F.Cu) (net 5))
 (segment (start 53.14 175.36) (end 53.14 175.36) (width 0.7) (layer F.Cu) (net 5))
 (via (at 53.14 175.36) (size 1.2) (drill 0.7) (layers F.Cu B.Cu) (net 5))
 (segment (start 48.77 179.73) (end 53.14 175.36) (width 0.7) (layer B.Cu) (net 5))
 (segment (start 41.88 184.54) (end 41.9 184.52) (width 0.55) (layer F.Cu) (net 5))
 (segment (start 35.1 184.54) (end 41.88 184.54) (width 0.55) (layer F.Cu) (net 5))
 (segment (start 41.9 184.52) (end 42.17 184.52) (width 0.55) (layer F.Cu) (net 5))
 (segment (start 48.77 179.73) (end 48.77 179.74) (width 0.55) (layer B.Cu) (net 5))
 (segment (start 45.1 179.22) (end 45.79 179.91) (width 0.7) (layer F.Cu) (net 5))
 (segment (start 43.71 182.71) (end 41.9 184.52) (width 0.7) (layer F.Cu) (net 5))
 (segment (start 43.842002 182.71) (end 43.862002 182.69) (width 0.7) (layer F.Cu) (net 5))
 (segment (start 43.71 182.71) (end 43.842002 182.71) (width 0.7) (layer F.Cu) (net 5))
 (segment (start 43.862002 182.69) (end 45.05 182.69) (width 0.7) (layer F.Cu) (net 5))
 (segment (start 45.79 181.95) (end 45.79 179.91) (width 0.7) (layer F.Cu) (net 5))
 (segment (start 45.05 182.69) (end 45.79 181.95) (width 0.7) (layer F.Cu) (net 5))
 (segment (start 48.77 179.73) (end 48.75 179.73) (width 0.7) (layer B.Cu) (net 5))
 (segment (start 48.75 179.73) (end 46.54 181.94) (width 0.7) (layer B.Cu) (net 5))
 (segment (start 46.54 181.94) (end 46.54 181.94) (width 0.7) (layer B.Cu) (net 5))
 (via (at 46.54 181.94) (size 1.2) (drill 0.7) (layers F.Cu B.Cu) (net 5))
 (segment (start 46.53 181.95) (end 46.54 181.94) (width 0.7) (layer F.Cu) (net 5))
 (segment (start 45.79 181.95) (end 46.53 181.95) (width 0.7) (layer F.Cu) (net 5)))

